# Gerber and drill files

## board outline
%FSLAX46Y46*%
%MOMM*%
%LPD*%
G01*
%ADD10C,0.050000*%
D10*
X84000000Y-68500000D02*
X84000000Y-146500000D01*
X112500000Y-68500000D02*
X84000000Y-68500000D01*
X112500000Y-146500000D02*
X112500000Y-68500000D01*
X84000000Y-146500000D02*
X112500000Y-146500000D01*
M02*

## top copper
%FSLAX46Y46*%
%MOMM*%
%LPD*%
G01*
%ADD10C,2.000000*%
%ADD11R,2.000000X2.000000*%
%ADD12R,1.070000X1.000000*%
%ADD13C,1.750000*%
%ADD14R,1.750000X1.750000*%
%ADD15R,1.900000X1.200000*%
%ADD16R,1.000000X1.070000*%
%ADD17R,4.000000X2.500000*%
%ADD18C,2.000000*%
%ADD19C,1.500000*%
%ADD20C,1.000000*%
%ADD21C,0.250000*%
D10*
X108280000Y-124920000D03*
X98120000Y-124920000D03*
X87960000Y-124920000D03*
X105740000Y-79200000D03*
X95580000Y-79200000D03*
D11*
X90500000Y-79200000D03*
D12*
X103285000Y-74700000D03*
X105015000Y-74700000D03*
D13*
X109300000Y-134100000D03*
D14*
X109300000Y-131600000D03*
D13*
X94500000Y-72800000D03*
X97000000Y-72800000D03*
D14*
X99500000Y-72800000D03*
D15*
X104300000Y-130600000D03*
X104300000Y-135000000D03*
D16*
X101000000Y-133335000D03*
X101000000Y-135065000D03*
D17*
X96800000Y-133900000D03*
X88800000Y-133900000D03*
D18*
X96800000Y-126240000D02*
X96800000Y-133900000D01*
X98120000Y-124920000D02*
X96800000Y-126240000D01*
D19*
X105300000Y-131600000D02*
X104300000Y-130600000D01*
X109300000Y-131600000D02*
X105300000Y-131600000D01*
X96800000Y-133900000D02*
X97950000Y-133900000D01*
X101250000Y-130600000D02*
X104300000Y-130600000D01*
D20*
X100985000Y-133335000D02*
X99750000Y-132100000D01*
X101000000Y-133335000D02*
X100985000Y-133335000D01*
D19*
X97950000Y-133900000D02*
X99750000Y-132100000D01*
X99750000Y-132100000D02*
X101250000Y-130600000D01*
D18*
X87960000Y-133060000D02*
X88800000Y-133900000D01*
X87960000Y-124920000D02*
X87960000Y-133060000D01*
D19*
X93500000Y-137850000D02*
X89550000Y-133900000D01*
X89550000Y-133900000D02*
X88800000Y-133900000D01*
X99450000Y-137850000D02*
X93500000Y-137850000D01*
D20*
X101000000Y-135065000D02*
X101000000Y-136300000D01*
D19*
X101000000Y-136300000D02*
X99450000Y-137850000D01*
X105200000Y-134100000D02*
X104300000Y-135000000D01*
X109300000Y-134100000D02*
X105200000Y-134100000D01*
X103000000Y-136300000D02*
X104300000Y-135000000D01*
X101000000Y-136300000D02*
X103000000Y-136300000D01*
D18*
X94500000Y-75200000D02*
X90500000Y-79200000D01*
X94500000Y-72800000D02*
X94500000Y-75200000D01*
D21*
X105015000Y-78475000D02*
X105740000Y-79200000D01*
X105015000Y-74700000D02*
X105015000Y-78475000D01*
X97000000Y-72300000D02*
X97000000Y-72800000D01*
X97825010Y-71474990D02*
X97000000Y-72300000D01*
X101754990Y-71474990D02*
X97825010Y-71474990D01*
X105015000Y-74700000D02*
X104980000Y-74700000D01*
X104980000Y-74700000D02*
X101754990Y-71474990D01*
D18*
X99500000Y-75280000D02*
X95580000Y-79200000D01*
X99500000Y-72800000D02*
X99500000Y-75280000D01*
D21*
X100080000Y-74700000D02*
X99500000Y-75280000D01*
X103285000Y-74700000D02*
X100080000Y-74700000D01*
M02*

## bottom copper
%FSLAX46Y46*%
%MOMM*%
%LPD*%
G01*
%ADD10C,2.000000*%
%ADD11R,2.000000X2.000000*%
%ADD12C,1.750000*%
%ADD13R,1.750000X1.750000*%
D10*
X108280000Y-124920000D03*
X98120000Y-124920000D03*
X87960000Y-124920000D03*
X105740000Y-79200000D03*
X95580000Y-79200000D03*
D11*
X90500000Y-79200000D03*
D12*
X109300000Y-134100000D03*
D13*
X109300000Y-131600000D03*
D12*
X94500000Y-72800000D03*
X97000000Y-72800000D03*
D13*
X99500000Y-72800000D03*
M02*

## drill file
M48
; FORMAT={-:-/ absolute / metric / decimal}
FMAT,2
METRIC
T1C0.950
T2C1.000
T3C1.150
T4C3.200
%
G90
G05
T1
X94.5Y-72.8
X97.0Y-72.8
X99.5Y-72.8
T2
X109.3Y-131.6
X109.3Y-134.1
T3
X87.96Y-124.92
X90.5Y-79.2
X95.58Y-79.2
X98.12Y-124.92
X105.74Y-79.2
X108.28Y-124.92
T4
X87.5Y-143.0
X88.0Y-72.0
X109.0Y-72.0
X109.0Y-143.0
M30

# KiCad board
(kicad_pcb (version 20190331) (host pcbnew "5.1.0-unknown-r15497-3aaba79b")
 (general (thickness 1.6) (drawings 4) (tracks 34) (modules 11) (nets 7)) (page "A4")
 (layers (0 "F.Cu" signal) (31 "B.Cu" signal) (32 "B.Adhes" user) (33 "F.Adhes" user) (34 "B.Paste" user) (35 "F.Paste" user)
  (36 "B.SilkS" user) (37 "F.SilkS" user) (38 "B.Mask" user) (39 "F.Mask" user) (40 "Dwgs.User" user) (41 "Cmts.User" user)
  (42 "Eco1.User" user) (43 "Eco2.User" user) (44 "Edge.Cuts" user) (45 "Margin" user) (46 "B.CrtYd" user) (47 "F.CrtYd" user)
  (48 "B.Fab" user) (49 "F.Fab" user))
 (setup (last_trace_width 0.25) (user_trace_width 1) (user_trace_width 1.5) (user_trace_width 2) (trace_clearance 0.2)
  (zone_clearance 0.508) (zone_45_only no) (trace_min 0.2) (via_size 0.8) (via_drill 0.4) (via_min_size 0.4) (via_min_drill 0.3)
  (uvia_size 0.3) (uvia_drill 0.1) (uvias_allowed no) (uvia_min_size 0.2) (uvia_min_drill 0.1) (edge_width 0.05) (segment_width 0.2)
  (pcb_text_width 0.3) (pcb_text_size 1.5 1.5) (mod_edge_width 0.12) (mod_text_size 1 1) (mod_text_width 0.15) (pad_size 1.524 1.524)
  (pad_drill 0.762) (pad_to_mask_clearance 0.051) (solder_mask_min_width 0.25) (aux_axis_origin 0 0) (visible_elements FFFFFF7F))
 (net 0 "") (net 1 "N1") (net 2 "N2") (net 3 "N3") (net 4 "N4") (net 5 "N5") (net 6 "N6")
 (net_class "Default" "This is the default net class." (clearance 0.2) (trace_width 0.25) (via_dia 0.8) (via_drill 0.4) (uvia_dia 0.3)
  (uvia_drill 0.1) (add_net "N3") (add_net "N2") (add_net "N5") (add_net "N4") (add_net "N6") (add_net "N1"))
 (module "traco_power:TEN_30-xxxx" (layer "F.Cu") (at 90.5 79.2)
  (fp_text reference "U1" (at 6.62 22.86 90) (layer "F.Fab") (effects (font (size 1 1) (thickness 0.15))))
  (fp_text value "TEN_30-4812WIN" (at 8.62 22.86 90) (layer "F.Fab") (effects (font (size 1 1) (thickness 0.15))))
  (pad "6" thru_hole circle (at 17.78 45.72) (size 2 2) (drill 1.15) (layers *.Cu *.Mask "F.SilkS") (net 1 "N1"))
  (pad "5" thru_hole circle (at 7.62 45.72) (size 2 2) (drill 1.15) (layers *.Cu *.Mask "F.SilkS") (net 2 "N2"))
  (pad "4" thru_hole circle (at -2.54 45.72) (size 2 2) (drill 1.15) (layers *.Cu *.Mask "F.SilkS") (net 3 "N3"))
  (pad "3" thru_hole circle (at 15.24 0) (size 2 2) (drill 1.15) (layers *.Cu *.Mask "F.SilkS") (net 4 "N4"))
  (pad "2" thru_hole circle (at 5.08 0) (size 2 2) (drill 1.15) (layers *.Cu *.Mask "F.SilkS") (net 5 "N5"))
  (pad "1" thru_hole rect (at 0 0) (size 2 2) (drill 1.15) (layers *.Cu *.Mask "F.SilkS") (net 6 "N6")))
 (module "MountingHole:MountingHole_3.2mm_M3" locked (layer "F.Cu") (at 87.5 143)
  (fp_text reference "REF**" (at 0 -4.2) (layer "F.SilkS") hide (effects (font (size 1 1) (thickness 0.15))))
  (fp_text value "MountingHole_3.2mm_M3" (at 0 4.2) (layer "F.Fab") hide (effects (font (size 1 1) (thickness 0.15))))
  (pad "1" np_thru_hole circle (at 0 0) (size 3.2 3.2) (drill 3.2) (layers *.Cu *.Mask)))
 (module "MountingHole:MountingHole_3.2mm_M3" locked (layer "F.Cu") (at 109 143)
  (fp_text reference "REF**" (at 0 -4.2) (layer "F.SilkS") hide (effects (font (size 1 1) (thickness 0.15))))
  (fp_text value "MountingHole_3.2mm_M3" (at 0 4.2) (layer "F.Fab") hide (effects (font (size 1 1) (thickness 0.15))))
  (pad "1" np_thru_hole circle (at 0 0) (size 3.2 3.2) (drill 3.2) (layers *.Cu *.Mask)))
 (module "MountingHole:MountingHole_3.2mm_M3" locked (layer "F.Cu") (at 88 72)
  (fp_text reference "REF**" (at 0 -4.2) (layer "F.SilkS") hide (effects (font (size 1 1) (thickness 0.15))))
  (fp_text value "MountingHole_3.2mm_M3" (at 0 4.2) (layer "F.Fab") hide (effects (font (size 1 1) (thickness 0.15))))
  (pad "1" np_thru_hole circle (at 0 0) (size 3.2 3.2) (drill 3.2) (layers *.Cu *.Mask)))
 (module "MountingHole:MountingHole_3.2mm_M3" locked (layer "F.Cu") (at 109 72)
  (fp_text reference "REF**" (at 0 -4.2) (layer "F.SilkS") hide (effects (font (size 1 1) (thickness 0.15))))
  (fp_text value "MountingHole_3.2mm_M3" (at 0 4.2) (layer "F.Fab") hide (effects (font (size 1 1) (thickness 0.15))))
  (pad "1" np_thru_hole circle (at 0 0) (size 3.2 3.2) (drill 3.2) (layers *.Cu *.Mask)))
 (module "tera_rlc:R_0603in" (layer "F.Cu") (at 104.15 74.7 180)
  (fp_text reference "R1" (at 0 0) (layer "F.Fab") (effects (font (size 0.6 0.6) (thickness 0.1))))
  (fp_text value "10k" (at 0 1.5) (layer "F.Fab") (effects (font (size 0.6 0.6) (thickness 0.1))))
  (pad "2" smd rect (at 0.865 0 180) (size 1.07 1) (layers "F.Cu" "F.Paste" "F.Mask") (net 5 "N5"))
  (pad "1" smd rect (at -0.865 0 180) (size 1.07 1) (layers "F.Cu" "F.Paste" "F.Mask") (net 4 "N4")))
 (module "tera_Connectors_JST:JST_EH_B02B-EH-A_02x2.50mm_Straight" (layer "F.Cu") (at 109.3 131.6 270)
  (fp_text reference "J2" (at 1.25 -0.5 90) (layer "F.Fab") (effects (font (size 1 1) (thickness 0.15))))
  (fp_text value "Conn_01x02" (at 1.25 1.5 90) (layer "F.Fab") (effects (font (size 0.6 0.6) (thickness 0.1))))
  (pad "2" thru_hole circle (at 2.5 0 270) (size 1.75 1.75) (drill 1) (layers *.Cu *.Mask) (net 3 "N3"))
  (pad "1" thru_hole rect (at 0 0 270) (size 1.75 1.75) (drill 1) (layers *.Cu *.Mask) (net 2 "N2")))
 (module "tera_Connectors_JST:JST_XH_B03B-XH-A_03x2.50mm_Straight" (layer "F.Cu") (at 99.5 72.8 180)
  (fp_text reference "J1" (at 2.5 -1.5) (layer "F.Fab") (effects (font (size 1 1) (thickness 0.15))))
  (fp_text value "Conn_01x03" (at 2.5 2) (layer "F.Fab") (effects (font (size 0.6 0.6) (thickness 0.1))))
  (pad "3" thru_hole circle (at 5 0 180) (size 1.75 1.75) (drill 0.95) (layers *.Cu *.Mask) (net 6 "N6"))
  (pad "2" thru_hole circle (at 2.5 0 180) (size 1.75 1.75) (drill 0.95) (layers *.Cu *.Mask) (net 4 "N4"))
  (pad "1" thru_hole rect (at 0 0 180) (size 1.75 1.75) (drill 0.95) (layers *.Cu *.Mask) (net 5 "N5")))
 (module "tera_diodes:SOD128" (layer "F.Cu") (at 104.3 132.8 90)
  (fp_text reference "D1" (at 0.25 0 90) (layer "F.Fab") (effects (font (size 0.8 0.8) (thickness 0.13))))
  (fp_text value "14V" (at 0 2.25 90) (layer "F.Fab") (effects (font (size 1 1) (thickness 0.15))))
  (pad "2" smd rect (at 2.2 0 90) (size 1.2 1.9) (layers "F.Cu" "F.Paste" "F.Mask") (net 2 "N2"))
  (pad "1" smd rect (at -2.2 0 90) (size 1.2 1.9) (layers "F.Cu" "F.Paste" "F.Mask") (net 3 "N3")))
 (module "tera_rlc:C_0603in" (layer "F.Cu") (at 101 134.2 90)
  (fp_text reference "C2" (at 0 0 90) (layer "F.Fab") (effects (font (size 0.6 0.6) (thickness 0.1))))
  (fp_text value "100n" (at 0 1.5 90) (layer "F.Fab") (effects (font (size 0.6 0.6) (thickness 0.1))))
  (pad "2" smd rect (at 0.865 0 90) (size 1.07 1) (layers "F.Cu" "F.Paste" "F.Mask") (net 2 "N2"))
  (pad "1" smd rect (at -0.865 0 90) (size 1.07 1) (layers "F.Cu" "F.Paste" "F.Mask") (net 3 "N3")))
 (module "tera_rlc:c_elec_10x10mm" (layer "F.Cu") (at 92.8 133.9)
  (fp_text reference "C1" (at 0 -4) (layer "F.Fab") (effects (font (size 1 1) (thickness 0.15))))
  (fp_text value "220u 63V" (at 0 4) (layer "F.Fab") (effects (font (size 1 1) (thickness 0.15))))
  (pad "2" smd rect (at 4 0 180) (size 4 2.5) (layers "F.Cu" "F.Paste" "F.Mask") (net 2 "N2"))
  (pad "1" smd rect (at -4 0 180) (size 4 2.5) (layers "F.Cu" "F.Paste" "F.Mask") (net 3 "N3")))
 (gr_line (start 84 68.5) (end 84 146.5) (layer "Edge.Cuts") (width 0.05))
 (gr_line (start 112.5 68.5) (end 84 68.5) (layer "Edge.Cuts") (width 0.05))
 (gr_line (start 112.5 146.5) (end 112.5 68.5) (layer "Edge.Cuts") (width 0.05))
 (gr_line (start 84 146.5) (end 112.5 146.5) (layer "Edge.Cuts") (width 0.05))
 (segment (start 96.8 126.24) (end 96.8 133.9) (width 2) (layer "F.Cu") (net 2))
 (segment (start 98.12 124.92) (end 96.8 126.24) (width 2) (layer "F.Cu") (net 2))
 (segment (start 105.3 131.6) (end 104.3 130.6) (width 1.5) (layer "F.Cu") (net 2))
 (segment (start 109.3 131.6) (end 105.3 131.6) (width 1.5) (layer "F.Cu") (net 2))
 (segment (start 96.8 133.9) (end 97.95 133.9) (width 1.5) (layer "F.Cu") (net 2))
 (segment (start 101.25 130.6) (end 104.3 130.6) (width 1.5) (layer "F.Cu") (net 2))
 (segment (start 100.985 133.335) (end 99.75 132.1) (width 1) (layer "F.Cu") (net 2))
 (segment (start 101 133.335) (end 100.985 133.335) (width 1) (layer "F.Cu") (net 2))
 (segment (start 97.95 133.9) (end 99.75 132.1) (width 1.5) (layer "F.Cu") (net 2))
 (segment (start 99.75 132.1) (end 101.25 130.6) (width 1.5) (layer "F.Cu") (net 2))
 (segment (start 87.96 133.06) (end 88.8 133.9) (width 2) (layer "F.Cu") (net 3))
 (segment (start 87.96 124.92) (end 87.96 133.06) (width 2) (layer "F.Cu") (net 3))
 (segment (start 93.5 137.85) (end 89.55 133.9) (width 1.5) (layer "F.Cu") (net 3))
 (segment (start 89.55 133.9) (end 88.8 133.9) (width 1.5) (layer "F.Cu") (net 3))
 (segment (start 99.45 137.85) (end 93.5 137.85) (width 1.5) (layer "F.Cu") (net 3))
 (segment (start 101 135.065) (end 101 136.3) (width 1) (layer "F.Cu") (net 3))
 (segment (start 101 136.3) (end 99.45 137.85) (width 1.5) (layer "F.Cu") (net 3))
 (segment (start 105.2 134.1) (end 104.3 135) (width 1.5) (layer "F.Cu") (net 3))
 (segment (start 109.3 134.1) (end 105.2 134.1) (width 1.5) (layer "F.Cu") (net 3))
 (segment (start 103 136.3) (end 104.3 135) (width 1.5) (layer "F.Cu") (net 3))
 (segment (start 101 136.3) (end 103 136.3) (width 1.5) (layer "F.Cu") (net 3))
 (segment (start 94.5 75.2) (end 90.5 79.2) (width 2) (layer "F.Cu") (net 6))
 (segment (start 94.5 72.8) (end 94.5 75.2) (width 2) (layer "F.Cu") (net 6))
 (segment (start 105.015 78.475) (end 105.74 79.2) (width 0.25) (layer "F.Cu") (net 4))
 (segment (start 105.015 74.7) (end 105.015 78.475) (width 0.25) (layer "F.Cu") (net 4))
 (segment (start 97 72.3) (end 97 72.8) (width 0.25) (layer "F.Cu") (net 4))
 (segment (start 97.82501 71.47499) (end 97 72.3) (width 0.25) (layer "F.Cu") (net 4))
 (segment (start 101.75499 71.47499) (end 97.82501 71.47499) (width 0.25) (layer "F.Cu") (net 4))
 (segment (start 105.015 74.7) (end 104.98 74.7) (width 0.25) (layer "F.Cu") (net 4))
 (segment (start 104.98 74.7) (end 101.75499 71.47499) (width 0.25) (layer "F.Cu") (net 4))
 (segment (start 99.5 75.28) (end 95.58 79.2) (width 2) (layer "F.Cu") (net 5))
 (segment (start 99.5 72.8) (end 99.5 75.28) (width 2) (layer "F.Cu") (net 5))
 (segment (start 100.08 74.7) (end 99.5 75.28) (width 0.25) (layer "F.Cu") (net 5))
 (segment (start 103.285 74.7) (end 100.08 74.7) (width 0.25) (layer "F.Cu") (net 5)))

